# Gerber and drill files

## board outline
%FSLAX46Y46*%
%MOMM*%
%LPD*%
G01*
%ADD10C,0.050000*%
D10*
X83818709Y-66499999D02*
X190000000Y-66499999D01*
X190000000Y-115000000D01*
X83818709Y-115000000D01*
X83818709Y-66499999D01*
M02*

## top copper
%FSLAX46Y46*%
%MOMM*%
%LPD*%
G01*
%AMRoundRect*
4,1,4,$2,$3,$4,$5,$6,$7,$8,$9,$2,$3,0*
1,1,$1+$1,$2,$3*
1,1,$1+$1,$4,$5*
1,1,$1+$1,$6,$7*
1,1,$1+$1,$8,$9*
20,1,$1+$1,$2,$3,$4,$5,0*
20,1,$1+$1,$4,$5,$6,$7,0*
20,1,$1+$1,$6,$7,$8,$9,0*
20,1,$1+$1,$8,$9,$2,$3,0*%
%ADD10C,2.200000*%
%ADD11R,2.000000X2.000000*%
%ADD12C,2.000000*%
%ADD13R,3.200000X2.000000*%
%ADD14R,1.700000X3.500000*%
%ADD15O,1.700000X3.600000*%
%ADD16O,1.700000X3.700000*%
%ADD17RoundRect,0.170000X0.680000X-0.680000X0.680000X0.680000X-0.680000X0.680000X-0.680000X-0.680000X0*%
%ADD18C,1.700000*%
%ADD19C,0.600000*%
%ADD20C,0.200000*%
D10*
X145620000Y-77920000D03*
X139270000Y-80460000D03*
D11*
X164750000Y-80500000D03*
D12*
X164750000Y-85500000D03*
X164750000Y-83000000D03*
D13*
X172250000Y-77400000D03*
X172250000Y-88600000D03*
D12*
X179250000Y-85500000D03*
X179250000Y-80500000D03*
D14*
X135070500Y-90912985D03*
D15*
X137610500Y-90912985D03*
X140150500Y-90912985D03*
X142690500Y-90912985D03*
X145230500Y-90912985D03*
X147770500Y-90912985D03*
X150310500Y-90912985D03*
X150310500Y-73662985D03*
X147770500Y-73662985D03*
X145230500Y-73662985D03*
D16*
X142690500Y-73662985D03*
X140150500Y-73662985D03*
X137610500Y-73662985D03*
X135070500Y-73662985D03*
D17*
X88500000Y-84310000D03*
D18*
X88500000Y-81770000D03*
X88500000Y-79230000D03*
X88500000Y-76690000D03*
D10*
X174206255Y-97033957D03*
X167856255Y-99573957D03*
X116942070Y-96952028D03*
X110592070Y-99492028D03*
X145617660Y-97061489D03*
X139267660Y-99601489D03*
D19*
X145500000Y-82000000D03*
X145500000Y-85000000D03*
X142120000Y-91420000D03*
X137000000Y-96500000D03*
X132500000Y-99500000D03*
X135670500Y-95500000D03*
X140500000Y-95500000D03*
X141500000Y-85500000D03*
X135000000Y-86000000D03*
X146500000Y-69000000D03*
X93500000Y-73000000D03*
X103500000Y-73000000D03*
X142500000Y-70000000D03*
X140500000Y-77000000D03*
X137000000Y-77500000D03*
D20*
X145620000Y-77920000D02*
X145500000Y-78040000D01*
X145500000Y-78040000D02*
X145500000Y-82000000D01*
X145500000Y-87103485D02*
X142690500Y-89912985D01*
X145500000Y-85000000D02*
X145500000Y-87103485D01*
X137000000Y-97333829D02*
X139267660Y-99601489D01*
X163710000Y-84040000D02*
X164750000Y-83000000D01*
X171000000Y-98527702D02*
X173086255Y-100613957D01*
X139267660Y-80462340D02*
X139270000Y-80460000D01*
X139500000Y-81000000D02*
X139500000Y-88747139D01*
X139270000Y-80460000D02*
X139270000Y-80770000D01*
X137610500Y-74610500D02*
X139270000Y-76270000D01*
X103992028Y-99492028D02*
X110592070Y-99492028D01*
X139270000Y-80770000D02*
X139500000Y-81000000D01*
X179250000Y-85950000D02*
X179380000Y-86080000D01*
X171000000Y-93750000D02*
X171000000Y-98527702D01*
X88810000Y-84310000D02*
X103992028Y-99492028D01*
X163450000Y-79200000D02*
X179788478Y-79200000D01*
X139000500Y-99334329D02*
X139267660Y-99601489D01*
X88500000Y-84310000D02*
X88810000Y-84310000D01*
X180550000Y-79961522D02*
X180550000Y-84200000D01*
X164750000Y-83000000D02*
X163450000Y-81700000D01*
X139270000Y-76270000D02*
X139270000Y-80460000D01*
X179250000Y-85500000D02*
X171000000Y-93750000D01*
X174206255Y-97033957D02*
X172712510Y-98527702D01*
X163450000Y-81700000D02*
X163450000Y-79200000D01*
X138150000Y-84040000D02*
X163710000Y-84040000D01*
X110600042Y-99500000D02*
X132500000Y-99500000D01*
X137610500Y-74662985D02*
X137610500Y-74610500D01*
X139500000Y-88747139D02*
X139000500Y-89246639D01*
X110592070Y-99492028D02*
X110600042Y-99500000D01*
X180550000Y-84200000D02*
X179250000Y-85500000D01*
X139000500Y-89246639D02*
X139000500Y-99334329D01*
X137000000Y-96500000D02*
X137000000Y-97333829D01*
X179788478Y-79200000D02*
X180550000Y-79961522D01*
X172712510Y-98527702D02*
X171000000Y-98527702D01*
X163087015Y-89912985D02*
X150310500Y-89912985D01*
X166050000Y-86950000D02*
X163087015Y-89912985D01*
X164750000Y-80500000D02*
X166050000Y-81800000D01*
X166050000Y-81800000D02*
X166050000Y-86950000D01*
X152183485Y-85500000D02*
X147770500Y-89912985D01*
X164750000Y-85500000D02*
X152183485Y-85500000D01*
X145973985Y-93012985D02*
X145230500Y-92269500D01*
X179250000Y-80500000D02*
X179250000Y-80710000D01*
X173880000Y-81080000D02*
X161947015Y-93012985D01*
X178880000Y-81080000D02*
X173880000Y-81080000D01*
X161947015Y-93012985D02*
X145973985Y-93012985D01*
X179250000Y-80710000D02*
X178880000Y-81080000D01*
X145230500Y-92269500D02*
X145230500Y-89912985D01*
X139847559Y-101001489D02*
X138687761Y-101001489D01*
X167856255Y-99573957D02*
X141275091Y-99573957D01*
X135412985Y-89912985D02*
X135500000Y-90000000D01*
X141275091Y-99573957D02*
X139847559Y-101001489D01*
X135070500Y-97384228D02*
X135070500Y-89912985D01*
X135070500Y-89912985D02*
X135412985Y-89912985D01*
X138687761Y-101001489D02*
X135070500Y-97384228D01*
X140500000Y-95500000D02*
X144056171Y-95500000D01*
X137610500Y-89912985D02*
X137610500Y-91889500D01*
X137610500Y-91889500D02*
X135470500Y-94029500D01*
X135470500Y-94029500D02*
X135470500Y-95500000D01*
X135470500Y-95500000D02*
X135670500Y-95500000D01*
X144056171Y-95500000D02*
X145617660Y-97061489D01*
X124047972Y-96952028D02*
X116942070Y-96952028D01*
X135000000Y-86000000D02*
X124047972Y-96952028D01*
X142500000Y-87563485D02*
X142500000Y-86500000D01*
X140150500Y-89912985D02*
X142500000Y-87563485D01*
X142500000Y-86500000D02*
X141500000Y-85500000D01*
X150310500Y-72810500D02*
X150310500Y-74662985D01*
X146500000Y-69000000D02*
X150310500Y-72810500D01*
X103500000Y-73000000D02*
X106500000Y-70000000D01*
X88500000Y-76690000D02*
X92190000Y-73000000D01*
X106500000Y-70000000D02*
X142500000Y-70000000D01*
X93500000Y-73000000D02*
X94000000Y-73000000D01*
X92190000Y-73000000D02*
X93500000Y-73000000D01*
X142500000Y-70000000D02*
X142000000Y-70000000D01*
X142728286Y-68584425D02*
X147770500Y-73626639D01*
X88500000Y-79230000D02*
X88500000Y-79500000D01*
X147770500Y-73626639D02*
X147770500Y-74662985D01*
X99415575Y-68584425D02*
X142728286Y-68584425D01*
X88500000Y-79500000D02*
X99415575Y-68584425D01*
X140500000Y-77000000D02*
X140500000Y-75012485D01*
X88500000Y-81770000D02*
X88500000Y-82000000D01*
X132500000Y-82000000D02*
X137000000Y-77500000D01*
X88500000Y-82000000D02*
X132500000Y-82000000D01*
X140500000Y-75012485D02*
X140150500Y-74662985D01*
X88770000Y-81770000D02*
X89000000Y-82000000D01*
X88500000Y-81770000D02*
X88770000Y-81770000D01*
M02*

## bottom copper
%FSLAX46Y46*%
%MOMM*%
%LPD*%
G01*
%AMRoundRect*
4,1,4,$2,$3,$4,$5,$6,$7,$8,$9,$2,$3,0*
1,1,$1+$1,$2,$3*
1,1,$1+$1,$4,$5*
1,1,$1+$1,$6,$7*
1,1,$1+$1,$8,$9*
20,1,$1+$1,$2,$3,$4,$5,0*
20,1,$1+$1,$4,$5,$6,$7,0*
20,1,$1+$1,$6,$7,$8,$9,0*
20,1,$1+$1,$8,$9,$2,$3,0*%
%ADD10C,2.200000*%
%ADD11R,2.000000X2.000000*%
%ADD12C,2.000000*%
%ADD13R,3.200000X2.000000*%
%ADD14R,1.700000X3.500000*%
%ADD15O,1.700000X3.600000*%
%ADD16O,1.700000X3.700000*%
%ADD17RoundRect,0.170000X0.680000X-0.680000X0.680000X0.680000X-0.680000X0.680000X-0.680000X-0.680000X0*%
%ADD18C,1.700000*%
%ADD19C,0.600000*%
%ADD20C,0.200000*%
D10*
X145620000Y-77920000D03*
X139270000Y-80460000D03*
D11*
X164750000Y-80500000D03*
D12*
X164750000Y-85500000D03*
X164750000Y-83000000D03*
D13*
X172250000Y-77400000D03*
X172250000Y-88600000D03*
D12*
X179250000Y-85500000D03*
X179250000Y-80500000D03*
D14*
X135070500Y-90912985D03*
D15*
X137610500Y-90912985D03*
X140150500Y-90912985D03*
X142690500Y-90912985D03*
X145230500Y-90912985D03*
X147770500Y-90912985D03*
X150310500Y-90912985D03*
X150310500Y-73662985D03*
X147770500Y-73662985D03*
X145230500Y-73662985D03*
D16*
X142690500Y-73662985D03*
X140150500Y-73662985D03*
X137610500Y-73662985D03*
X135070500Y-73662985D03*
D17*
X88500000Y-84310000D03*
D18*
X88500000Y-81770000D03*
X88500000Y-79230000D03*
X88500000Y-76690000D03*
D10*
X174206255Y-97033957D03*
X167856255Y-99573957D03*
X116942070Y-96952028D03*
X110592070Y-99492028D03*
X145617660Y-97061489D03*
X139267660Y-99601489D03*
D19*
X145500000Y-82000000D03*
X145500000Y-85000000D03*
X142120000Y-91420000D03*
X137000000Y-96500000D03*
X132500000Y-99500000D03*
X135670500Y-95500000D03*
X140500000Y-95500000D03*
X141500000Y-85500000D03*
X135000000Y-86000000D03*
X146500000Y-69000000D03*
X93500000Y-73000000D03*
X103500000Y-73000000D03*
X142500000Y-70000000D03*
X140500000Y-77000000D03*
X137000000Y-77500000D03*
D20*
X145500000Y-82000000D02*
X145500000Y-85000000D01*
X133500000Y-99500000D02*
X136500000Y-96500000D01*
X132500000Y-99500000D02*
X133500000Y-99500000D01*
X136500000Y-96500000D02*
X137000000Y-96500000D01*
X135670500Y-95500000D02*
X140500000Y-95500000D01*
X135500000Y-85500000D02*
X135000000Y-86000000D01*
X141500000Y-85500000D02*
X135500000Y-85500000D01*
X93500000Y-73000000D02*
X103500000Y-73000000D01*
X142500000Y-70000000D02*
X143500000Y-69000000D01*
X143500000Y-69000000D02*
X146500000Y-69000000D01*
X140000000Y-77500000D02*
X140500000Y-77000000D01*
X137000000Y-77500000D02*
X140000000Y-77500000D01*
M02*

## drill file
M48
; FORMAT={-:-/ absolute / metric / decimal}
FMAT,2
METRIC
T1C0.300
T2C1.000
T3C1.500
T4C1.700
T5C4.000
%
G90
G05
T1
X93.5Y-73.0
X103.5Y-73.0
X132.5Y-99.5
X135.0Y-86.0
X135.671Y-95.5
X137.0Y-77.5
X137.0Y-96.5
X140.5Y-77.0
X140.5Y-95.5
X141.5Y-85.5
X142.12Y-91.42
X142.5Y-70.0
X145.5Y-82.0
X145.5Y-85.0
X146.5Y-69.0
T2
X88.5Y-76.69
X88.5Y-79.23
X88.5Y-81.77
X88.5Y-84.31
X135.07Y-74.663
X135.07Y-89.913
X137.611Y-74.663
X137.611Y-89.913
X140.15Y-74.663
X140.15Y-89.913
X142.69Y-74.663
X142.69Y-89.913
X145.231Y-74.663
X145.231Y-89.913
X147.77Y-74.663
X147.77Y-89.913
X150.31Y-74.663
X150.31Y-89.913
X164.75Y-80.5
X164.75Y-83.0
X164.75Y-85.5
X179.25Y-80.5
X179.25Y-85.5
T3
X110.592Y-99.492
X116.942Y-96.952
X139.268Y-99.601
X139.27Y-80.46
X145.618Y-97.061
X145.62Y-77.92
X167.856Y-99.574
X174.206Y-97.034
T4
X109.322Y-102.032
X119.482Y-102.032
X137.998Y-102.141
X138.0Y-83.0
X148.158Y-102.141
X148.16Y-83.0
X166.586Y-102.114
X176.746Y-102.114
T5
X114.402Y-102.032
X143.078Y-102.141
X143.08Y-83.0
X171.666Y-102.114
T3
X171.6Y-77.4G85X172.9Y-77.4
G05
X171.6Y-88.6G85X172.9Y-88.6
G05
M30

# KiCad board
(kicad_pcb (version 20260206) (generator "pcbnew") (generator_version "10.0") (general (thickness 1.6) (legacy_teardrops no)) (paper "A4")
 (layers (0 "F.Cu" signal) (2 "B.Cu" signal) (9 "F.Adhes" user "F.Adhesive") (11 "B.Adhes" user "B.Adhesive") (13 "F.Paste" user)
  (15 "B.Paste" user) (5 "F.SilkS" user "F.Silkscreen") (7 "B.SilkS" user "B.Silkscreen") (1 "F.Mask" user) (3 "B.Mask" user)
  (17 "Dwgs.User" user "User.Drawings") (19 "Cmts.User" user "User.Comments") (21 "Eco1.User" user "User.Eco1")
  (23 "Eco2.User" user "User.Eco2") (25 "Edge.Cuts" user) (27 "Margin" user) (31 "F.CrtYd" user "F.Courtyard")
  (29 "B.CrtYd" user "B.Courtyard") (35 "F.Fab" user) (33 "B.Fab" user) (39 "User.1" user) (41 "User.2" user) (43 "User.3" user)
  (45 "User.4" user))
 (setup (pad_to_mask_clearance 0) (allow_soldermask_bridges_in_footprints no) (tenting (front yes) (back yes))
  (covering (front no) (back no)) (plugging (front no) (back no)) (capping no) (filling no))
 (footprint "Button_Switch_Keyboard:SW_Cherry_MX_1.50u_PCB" (layer "F.Cu") (at 145.62 77.92)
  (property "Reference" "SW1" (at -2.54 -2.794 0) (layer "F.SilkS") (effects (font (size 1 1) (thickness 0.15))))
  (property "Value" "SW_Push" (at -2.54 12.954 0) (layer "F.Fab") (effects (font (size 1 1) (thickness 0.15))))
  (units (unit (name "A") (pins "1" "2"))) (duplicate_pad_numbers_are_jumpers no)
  (pad "" np_thru_hole circle (at -7.62 5.08) (size 1.7 1.7) (drill 1.7) (layers "*.Cu" "*.Mask"))
  (pad "" np_thru_hole circle (at -2.54 5.08) (size 4 4) (drill 4) (layers "*.Cu" "*.Mask"))
  (pad "" np_thru_hole circle (at 2.54 5.08) (size 1.7 1.7) (drill 1.7) (layers "*.Cu" "*.Mask"))
  (pad "1" thru_hole circle (at 0 0) (size 2.2 2.2) (drill 1.5) (layers "*.Cu" "*.Mask") (remove_unused_layers no)
   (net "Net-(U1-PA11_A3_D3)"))
  (pad "2" thru_hole circle (at -6.35 2.54) (size 2.2 2.2) (drill 1.5) (layers "*.Cu" "*.Mask") (remove_unused_layers no) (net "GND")))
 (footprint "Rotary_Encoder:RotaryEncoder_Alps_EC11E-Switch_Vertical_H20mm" (layer "F.Cu") (at 164.75 80.5)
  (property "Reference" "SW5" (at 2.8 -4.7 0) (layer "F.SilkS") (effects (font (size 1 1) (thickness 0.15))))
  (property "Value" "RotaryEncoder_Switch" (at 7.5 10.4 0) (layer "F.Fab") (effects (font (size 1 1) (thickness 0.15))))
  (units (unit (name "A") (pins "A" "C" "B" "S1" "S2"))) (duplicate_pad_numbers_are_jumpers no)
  (pad "A" thru_hole rect (at 0 0) (size 2 2) (drill 1) (layers "*.Cu" "*.Mask") (remove_unused_layers no) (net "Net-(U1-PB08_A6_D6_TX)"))
  (pad "B" thru_hole circle (at 0 5) (size 2 2) (drill 1) (layers "*.Cu" "*.Mask") (remove_unused_layers no) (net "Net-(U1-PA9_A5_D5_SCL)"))
  (pad "C" thru_hole circle (at 0 2.5) (size 2 2) (drill 1) (layers "*.Cu" "*.Mask") (remove_unused_layers no) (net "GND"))
  (pad "MP" thru_hole rect (at 7.5 -3.1) (size 3.2 2) (drill oval 2.8 1.5) (layers "*.Cu" "*.Mask") (remove_unused_layers no))
  (pad "MP" thru_hole rect (at 7.5 8.1) (size 3.2 2) (drill oval 2.8 1.5) (layers "*.Cu" "*.Mask") (remove_unused_layers no))
  (pad "S1" thru_hole circle (at 14.5 5) (size 2 2) (drill 1) (layers "*.Cu" "*.Mask") (remove_unused_layers no) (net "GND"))
  (pad "S2" thru_hole circle (at 14.5 0) (size 2 2) (drill 1) (layers "*.Cu" "*.Mask") (remove_unused_layers no)
   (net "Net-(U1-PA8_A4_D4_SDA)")))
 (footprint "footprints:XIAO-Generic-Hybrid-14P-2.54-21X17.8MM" (layer "F.Cu") (at 142.6905 82.287985 90)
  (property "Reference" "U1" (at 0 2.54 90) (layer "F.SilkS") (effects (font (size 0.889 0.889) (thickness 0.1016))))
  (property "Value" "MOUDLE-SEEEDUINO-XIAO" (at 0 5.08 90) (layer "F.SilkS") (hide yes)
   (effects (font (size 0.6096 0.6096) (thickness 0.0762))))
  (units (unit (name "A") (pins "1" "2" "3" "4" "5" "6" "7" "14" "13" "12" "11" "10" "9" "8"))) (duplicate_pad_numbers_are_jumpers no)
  (pad "1" thru_hole rect (at -7.625 -7.62 90) (size 3.5 1.7) (drill 1 (offset -1 0)) (layers "*.Cu" "*.Mask") (remove_unused_layers no)
   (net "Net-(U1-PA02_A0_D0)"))
  (pad "2" thru_hole oval (at -7.625 -5.08 90) (size 3.6 1.7) (drill 1 (offset -1 0)) (layers "*.Cu" "*.Mask") (remove_unused_layers no)
   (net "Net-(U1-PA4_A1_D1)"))
  (pad "3" thru_hole oval (at -7.625 -2.54 90) (size 3.6 1.7) (drill 1 (offset -1 0)) (layers "*.Cu" "*.Mask") (remove_unused_layers no)
   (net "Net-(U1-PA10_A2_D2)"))
  (pad "4" thru_hole oval (at -7.625 0 90) (size 3.6 1.7) (drill 1 (offset -1 0)) (layers "*.Cu" "*.Mask") (remove_unused_layers no)
   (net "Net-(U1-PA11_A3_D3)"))
  (pad "5" thru_hole oval (at -7.625 2.54 90) (size 3.6 1.7) (drill 1 (offset -1 0)) (layers "*.Cu" "*.Mask") (remove_unused_layers no)
   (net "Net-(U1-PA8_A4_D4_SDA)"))
  (pad "6" thru_hole oval (at -7.625 5.08 270) (size 3.6 1.7) (drill 1 (offset 1 0)) (layers "*.Cu" "*.Mask") (remove_unused_layers no)
   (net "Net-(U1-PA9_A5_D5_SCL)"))
  (pad "7" thru_hole oval (at -7.625 7.62 90) (size 3.6 1.7) (drill 1 (offset -1 0)) (layers "*.Cu" "*.Mask") (remove_unused_layers no)
   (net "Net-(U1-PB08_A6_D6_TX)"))
  (pad "8" thru_hole oval (at 7.625 7.62 90) (size 3.6 1.7) (drill 1 (offset 1 0)) (layers "*.Cu" "*.Mask") (remove_unused_layers no)
   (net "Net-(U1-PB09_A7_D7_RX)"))
  (pad "9" thru_hole oval (at 7.625 5.08 90) (size 3.6 1.7) (drill 1 (offset 1 0)) (layers "*.Cu" "*.Mask") (remove_unused_layers no)
   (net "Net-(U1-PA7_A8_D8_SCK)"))
  (pad "10" thru_hole oval (at 7.625 2.54 90) (size 3.6 1.7) (drill 1 (offset 1 0)) (layers "*.Cu" "*.Mask") (remove_unused_layers no)
   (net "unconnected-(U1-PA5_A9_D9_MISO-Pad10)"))
  (pad "11" thru_hole oval (at 7.625 0 90) (size 3.7 1.7) (drill 1 (offset 1 0)) (layers "*.Cu" "*.Mask") (remove_unused_layers no)
   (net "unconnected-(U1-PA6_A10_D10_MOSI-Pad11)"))
  (pad "12" thru_hole oval (at 7.625 -2.54 90) (size 3.7 1.7) (drill 1 (offset 1 0)) (layers "*.Cu" "*.Mask") (remove_unused_layers no)
   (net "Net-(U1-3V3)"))
  (pad "13" thru_hole oval (at 7.625 -5.08 90) (size 3.7 1.7) (drill 1 (offset 1 0)) (layers "*.Cu" "*.Mask") (remove_unused_layers no)
   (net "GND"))
  (pad "14" thru_hole oval (at 7.625 -7.62 90) (size 3.7 1.7) (drill 1 (offset 1 0)) (layers "*.Cu" "*.Mask") (remove_unused_layers no)
   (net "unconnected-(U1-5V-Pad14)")))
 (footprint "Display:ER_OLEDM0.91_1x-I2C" (layer "F.Cu") (at 88.5 84.31 90)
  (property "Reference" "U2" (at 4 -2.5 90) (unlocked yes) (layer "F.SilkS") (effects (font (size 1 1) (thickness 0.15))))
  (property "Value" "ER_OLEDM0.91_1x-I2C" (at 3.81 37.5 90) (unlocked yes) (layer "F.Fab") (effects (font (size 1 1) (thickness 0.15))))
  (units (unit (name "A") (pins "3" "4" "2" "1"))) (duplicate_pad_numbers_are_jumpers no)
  (pad "1" thru_hole roundrect (at 0 0 90) (size 1.7 1.7) (drill 1) (layers "*.Cu" "*.Mask") (remove_unused_layers no)
   (roundrect_rratio 0.1) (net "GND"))
  (pad "2" thru_hole circle (at 2.54 0 90) (size 1.7 1.7) (drill 1) (layers "*.Cu" "*.Mask") (remove_unused_layers no) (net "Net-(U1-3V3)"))
  (pad "3" thru_hole circle (at 5.08 0 90) (size 1.7 1.7) (drill 1) (layers "*.Cu" "*.Mask") (remove_unused_layers no)
   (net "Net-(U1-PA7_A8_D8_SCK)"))
  (pad "4" thru_hole circle (at 7.62 0 90) (size 1.7 1.7) (drill 1) (layers "*.Cu" "*.Mask") (remove_unused_layers no)
   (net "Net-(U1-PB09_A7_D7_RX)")))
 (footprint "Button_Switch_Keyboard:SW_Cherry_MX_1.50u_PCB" (layer "F.Cu") (at 174.206255 97.033957)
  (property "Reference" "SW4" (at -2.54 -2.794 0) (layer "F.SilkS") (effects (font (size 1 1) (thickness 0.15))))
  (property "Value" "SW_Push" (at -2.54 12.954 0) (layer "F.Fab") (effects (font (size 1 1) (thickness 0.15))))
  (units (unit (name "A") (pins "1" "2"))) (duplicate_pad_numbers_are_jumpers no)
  (pad "" np_thru_hole circle (at -7.62 5.08) (size 1.7 1.7) (drill 1.7) (layers "*.Cu" "*.Mask"))
  (pad "" np_thru_hole circle (at -2.54 5.08) (size 4 4) (drill 4) (layers "*.Cu" "*.Mask"))
  (pad "" np_thru_hole circle (at 2.54 5.08) (size 1.7 1.7) (drill 1.7) (layers "*.Cu" "*.Mask"))
  (pad "1" thru_hole circle (at 0 0) (size 2.2 2.2) (drill 1.5) (layers "*.Cu" "*.Mask") (remove_unused_layers no) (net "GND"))
  (pad "2" thru_hole circle (at -6.35 2.54) (size 2.2 2.2) (drill 1.5) (layers "*.Cu" "*.Mask") (remove_unused_layers no)
   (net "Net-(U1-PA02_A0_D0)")))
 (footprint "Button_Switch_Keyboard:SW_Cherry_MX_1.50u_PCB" (layer "F.Cu") (at 116.94207 96.952028)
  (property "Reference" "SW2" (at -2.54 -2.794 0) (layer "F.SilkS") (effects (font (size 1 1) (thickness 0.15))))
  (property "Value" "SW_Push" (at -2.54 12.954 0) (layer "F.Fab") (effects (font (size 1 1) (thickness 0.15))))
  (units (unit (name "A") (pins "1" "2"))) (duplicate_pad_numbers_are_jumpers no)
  (pad "" np_thru_hole circle (at -7.62 5.08) (size 1.7 1.7) (drill 1.7) (layers "*.Cu" "*.Mask"))
  (pad "" np_thru_hole circle (at -2.54 5.08) (size 4 4) (drill 4) (layers "*.Cu" "*.Mask"))
  (pad "" np_thru_hole circle (at 2.54 5.08) (size 1.7 1.7) (drill 1.7) (layers "*.Cu" "*.Mask"))
  (pad "1" thru_hole circle (at 0 0) (size 2.2 2.2) (drill 1.5) (layers "*.Cu" "*.Mask") (remove_unused_layers no)
   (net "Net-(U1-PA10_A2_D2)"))
  (pad "2" thru_hole circle (at -6.35 2.54) (size 2.2 2.2) (drill 1.5) (layers "*.Cu" "*.Mask") (remove_unused_layers no) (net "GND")))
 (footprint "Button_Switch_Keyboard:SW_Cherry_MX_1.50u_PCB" (layer "F.Cu") (at 145.61766 97.061489)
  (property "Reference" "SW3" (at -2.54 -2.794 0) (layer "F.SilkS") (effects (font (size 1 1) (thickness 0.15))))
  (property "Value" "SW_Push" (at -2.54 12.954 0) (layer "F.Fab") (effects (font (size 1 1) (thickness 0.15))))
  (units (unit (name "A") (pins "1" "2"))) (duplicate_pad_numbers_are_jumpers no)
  (pad "" np_thru_hole circle (at -7.62 5.08) (size 1.7 1.7) (drill 1.7) (layers "*.Cu" "*.Mask"))
  (pad "" np_thru_hole circle (at -2.54 5.08) (size 4 4) (drill 4) (layers "*.Cu" "*.Mask"))
  (pad "" np_thru_hole circle (at 2.54 5.08) (size 1.7 1.7) (drill 1.7) (layers "*.Cu" "*.Mask"))
  (pad "1" thru_hole circle (at 0 0) (size 2.2 2.2) (drill 1.5) (layers "*.Cu" "*.Mask") (remove_unused_layers no)
   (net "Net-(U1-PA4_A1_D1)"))
  (pad "2" thru_hole circle (at -6.35 2.54) (size 2.2 2.2) (drill 1.5) (layers "*.Cu" "*.Mask") (remove_unused_layers no) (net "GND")))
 (gr_rect (start 83.818709 66.499999) (end 190 115) (stroke (width 0.05) (type default)) (fill no) (layer "Edge.Cuts"))
 (segment (start 145.62 77.92) (end 145.5 78.04) (width 0.2) (layer "F.Cu") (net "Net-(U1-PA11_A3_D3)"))
 (segment (start 145.5 78.04) (end 145.5 82) (width 0.2) (layer "F.Cu") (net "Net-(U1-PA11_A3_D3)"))
 (segment (start 145.5 87.103485) (end 142.6905 89.912985) (width 0.2) (layer "F.Cu") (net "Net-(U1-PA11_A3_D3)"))
 (segment (start 145.5 85) (end 145.5 87.103485) (width 0.2) (layer "F.Cu") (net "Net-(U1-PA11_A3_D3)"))
 (via (at 145.5 82) (size 0.6) (drill 0.3) (layers "F.Cu" "B.Cu") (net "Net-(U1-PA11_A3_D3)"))
 (via (at 145.5 85) (size 0.6) (drill 0.3) (layers "F.Cu" "B.Cu") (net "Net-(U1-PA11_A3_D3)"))
 (via (at 142.12 91.42) (size 0.6) (drill 0.3) (layers "F.Cu" "B.Cu") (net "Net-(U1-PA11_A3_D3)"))
 (segment (start 145.5 82) (end 145.5 85) (width 0.2) (layer "B.Cu") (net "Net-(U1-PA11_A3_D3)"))
 (segment (start 137 97.333829) (end 139.26766 99.601489) (width 0.2) (layer "F.Cu") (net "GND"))
 (segment (start 163.71 84.04) (end 164.75 83) (width 0.2) (layer "F.Cu") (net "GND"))
 (segment (start 171 98.527702) (end 173.086255 100.613957) (width 0.2) (layer "F.Cu") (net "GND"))
 (segment (start 139.26766 80.46234) (end 139.27 80.46) (width 0.2) (layer "F.Cu") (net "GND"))
 (segment (start 139.5 81) (end 139.5 88.747139) (width 0.2) (layer "F.Cu") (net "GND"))
 (segment (start 139.27 80.46) (end 139.27 80.77) (width 0.2) (layer "F.Cu") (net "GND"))
 (segment (start 137.6105 74.6105) (end 139.27 76.27) (width 0.2) (layer "F.Cu") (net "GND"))
 (segment (start 103.992028 99.492028) (end 110.59207 99.492028) (width 0.2) (layer "F.Cu") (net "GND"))
 (segment (start 139.27 80.77) (end 139.5 81) (width 0.2) (layer "F.Cu") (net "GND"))
 (segment (start 179.25 85.95) (end 179.38 86.08) (width 0.2) (layer "F.Cu") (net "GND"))
 (segment (start 171 93.75) (end 171 98.527702) (width 0.2) (layer "F.Cu") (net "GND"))
 (segment (start 88.81 84.31) (end 103.992028 99.492028) (width 0.2) (layer "F.Cu") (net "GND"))
 (segment (start 163.45 79.2) (end 179.788478 79.2) (width 0.2) (layer "F.Cu") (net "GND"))
 (segment (start 139.0005 99.334329) (end 139.26766 99.601489) (width 0.2) (layer "F.Cu") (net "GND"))
 (segment (start 88.5 84.31) (end 88.81 84.31) (width 0.2) (layer "F.Cu") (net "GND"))
 (segment (start 180.55 79.961522) (end 180.55 84.2) (width 0.2) (layer "F.Cu") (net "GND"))
 (segment (start 164.75 83) (end 163.45 81.7) (width 0.2) (layer "F.Cu") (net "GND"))
 (segment (start 139.27 76.27) (end 139.27 80.46) (width 0.2) (layer "F.Cu") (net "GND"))
 (segment (start 179.25 85.5) (end 171 93.75) (width 0.2) (layer "F.Cu") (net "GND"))
 (segment (start 174.206255 97.033957) (end 172.71251 98.527702) (width 0.2) (layer "F.Cu") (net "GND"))
 (segment (start 163.45 81.7) (end 163.45 79.2) (width 0.2) (layer "F.Cu") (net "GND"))
 (segment (start 138.15 84.04) (end 163.71 84.04) (width 0.2) (layer "F.Cu") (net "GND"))
 (segment (start 110.600042 99.5) (end 132.5 99.5) (width 0.2) (layer "F.Cu") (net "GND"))
 (segment (start 137.6105 74.662985) (end 137.6105 74.6105) (width 0.2) (layer "F.Cu") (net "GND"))
 (segment (start 139.5 88.747139) (end 139.0005 89.246639) (width 0.2) (layer "F.Cu") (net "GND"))
 (segment (start 110.59207 99.492028) (end 110.600042 99.5) (width 0.2) (layer "F.Cu") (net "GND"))
 (segment (start 180.55 84.2) (end 179.25 85.5) (width 0.2) (layer "F.Cu") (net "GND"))
 (segment (start 139.0005 89.246639) (end 139.0005 99.334329) (width 0.2) (layer "F.Cu") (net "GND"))
 (segment (start 137 96.5) (end 137 97.333829) (width 0.2) (layer "F.Cu") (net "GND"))
 (segment (start 179.788478 79.2) (end 180.55 79.961522) (width 0.2) (layer "F.Cu") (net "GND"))
 (segment (start 172.71251 98.527702) (end 171 98.527702) (width 0.2) (layer "F.Cu") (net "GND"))
 (via (at 137 96.5) (size 0.6) (drill 0.3) (layers "F.Cu" "B.Cu") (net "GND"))
 (via (at 132.5 99.5) (size 0.6) (drill 0.3) (layers "F.Cu" "B.Cu") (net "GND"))
 (segment (start 133.5 99.5) (end 136.5 96.5) (width 0.2) (layer "B.Cu") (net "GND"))
 (segment (start 132.5 99.5) (end 133.5 99.5) (width 0.2) (layer "B.Cu") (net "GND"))
 (segment (start 136.5 96.5) (end 137 96.5) (width 0.2) (layer "B.Cu") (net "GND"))
 (segment (start 163.087015 89.912985) (end 150.3105 89.912985) (width 0.2) (layer "F.Cu") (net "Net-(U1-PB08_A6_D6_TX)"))
 (segment (start 166.05 86.95) (end 163.087015 89.912985) (width 0.2) (layer "F.Cu") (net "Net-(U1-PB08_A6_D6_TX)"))
 (segment (start 164.75 80.5) (end 166.05 81.8) (width 0.2) (layer "F.Cu") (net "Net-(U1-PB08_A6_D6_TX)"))
 (segment (start 166.05 81.8) (end 166.05 86.95) (width 0.2) (layer "F.Cu") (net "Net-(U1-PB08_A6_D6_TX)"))
 (segment (start 152.183485 85.5) (end 147.7705 89.912985) (width 0.2) (layer "F.Cu") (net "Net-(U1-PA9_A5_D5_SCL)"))
 (segment (start 164.75 85.5) (end 152.183485 85.5) (width 0.2) (layer "F.Cu") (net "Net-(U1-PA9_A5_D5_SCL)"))
 (segment (start 145.973985 93.012985) (end 145.2305 92.2695) (width 0.2) (layer "F.Cu") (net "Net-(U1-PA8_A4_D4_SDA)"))
 (segment (start 179.25 80.5) (end 179.25 80.71) (width 0.2) (layer "F.Cu") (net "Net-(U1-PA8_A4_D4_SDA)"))
 (segment (start 173.88 81.08) (end 161.947015 93.012985) (width 0.2) (layer "F.Cu") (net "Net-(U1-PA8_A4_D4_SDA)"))
 (segment (start 178.88 81.08) (end 173.88 81.08) (width 0.2) (layer "F.Cu") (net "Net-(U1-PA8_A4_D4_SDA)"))
 (segment (start 161.947015 93.012985) (end 145.973985 93.012985) (width 0.2) (layer "F.Cu") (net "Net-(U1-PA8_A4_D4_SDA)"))
 (segment (start 179.25 80.71) (end 178.88 81.08) (width 0.2) (layer "F.Cu") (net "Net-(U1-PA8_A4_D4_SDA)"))
 (segment (start 145.2305 92.2695) (end 145.2305 89.912985) (width 0.2) (layer "F.Cu") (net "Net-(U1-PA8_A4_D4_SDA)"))
 (segment (start 139.847559 101.001489) (end 138.687761 101.001489) (width 0.2) (layer "F.Cu") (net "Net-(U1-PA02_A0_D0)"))
 (segment (start 167.856255 99.573957) (end 141.275091 99.573957) (width 0.2) (layer "F.Cu") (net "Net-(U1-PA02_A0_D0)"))
 (segment (start 135.412985 89.912985) (end 135.5 90) (width 0.2) (layer "F.Cu") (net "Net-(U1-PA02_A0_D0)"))
 (segment (start 141.275091 99.573957) (end 139.847559 101.001489) (width 0.2) (layer "F.Cu") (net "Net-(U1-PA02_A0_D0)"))
 (segment (start 135.0705 97.384228) (end 135.0705 89.912985) (width 0.2) (layer "F.Cu") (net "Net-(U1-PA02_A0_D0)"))
 (segment (start 135.0705 89.912985) (end 135.412985 89.912985) (width 0.2) (layer "F.Cu") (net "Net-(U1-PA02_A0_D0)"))
 (segment (start 138.687761 101.001489) (end 135.0705 97.384228) (width 0.2) (layer "F.Cu") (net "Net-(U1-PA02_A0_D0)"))
 (segment (start 140.5 95.5) (end 144.056171 95.5) (width 0.2) (layer "F.Cu") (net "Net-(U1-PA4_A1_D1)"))
 (segment (start 137.6105 89.912985) (end 137.6105 91.8895) (width 0.2) (layer "F.Cu") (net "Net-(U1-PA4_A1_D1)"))
 (segment (start 137.6105 91.8895) (end 135.4705 94.0295) (width 0.2) (layer "F.Cu") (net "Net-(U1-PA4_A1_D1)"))
 (segment (start 135.4705 94.0295) (end 135.4705 95.5) (width 0.2) (layer "F.Cu") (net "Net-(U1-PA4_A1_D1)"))
 (segment (start 135.4705 95.5) (end 135.6705 95.5) (width 0.2) (layer "F.Cu") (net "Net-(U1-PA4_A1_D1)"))
 (segment (start 144.056171 95.5) (end 145.61766 97.061489) (width 0.2) (layer "F.Cu") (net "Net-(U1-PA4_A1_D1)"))
 (via (at 135.6705 95.5) (size 0.6) (drill 0.3) (layers "F.Cu" "B.Cu") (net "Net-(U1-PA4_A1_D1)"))
 (via (at 140.5 95.5) (size 0.6) (drill 0.3) (layers "F.Cu" "B.Cu") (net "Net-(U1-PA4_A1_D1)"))
 (segment (start 135.6705 95.5) (end 140.5 95.5) (width 0.2) (layer "B.Cu") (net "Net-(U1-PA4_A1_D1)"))
 (segment (start 124.047972 96.952028) (end 116.94207 96.952028) (width 0.2) (layer "F.Cu") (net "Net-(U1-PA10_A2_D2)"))
 (segment (start 135 86) (end 124.047972 96.952028) (width 0.2) (layer "F.Cu") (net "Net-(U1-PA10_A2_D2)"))
 (segment (start 142.5 87.563485) (end 142.5 86.5) (width 0.2) (layer "F.Cu") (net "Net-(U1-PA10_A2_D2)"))
 (segment (start 140.1505 89.912985) (end 142.5 87.563485) (width 0.2) (layer "F.Cu") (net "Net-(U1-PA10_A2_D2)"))
 (segment (start 142.5 86.5) (end 141.5 85.5) (width 0.2) (layer "F.Cu") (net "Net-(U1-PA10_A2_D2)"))
 (via (at 141.5 85.5) (size 0.6) (drill 0.3) (layers "F.Cu" "B.Cu") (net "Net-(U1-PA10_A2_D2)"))
 (via (at 135 86) (size 0.6) (drill 0.3) (layers "F.Cu" "B.Cu") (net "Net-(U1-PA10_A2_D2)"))
 (segment (start 135.5 85.5) (end 135 86) (width 0.2) (layer "B.Cu") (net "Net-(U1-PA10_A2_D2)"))
 (segment (start 141.5 85.5) (end 135.5 85.5) (width 0.2) (layer "B.Cu") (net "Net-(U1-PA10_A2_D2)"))
 (segment (start 150.3105 72.8105) (end 150.3105 74.662985) (width 0.2) (layer "F.Cu") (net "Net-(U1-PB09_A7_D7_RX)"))
 (segment (start 146.5 69) (end 150.3105 72.8105) (width 0.2) (layer "F.Cu") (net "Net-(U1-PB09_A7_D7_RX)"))
 (segment (start 103.5 73) (end 106.5 70) (width 0.2) (layer "F.Cu") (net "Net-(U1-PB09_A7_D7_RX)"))
 (segment (start 88.5 76.69) (end 92.19 73) (width 0.2) (layer "F.Cu") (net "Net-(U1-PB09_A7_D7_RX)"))
 (segment (start 106.5 70) (end 142.5 70) (width 0.2) (layer "F.Cu") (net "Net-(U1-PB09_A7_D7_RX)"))
 (segment (start 93.5 73) (end 94 73) (width 0.2) (layer "F.Cu") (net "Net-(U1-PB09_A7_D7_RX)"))
 (segment (start 92.19 73) (end 93.5 73) (width 0.2) (layer "F.Cu") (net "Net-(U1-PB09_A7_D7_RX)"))
 (segment (start 142.5 70) (end 142 70) (width 0.2) (layer "F.Cu") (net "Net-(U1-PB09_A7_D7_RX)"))
 (via (at 146.5 69) (size 0.6) (drill 0.3) (layers "F.Cu" "B.Cu") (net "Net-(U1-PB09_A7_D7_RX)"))
 (via (at 93.5 73) (size 0.6) (drill 0.3) (layers "F.Cu" "B.Cu") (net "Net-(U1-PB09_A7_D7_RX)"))
 (via (at 103.5 73) (size 0.6) (drill 0.3) (layers "F.Cu" "B.Cu") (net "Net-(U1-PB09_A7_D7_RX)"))
 (via (at 142.5 70) (size 0.6) (drill 0.3) (layers "F.Cu" "B.Cu") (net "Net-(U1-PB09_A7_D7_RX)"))
 (segment (start 93.5 73) (end 103.5 73) (width 0.2) (layer "B.Cu") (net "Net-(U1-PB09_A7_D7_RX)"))
 (segment (start 142.5 70) (end 143.5 69) (width 0.2) (layer "B.Cu") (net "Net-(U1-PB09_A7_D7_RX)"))
 (segment (start 143.5 69) (end 146.5 69) (width 0.2) (layer "B.Cu") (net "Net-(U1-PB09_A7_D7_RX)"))
 (segment (start 142.728286 68.584425) (end 147.7705 73.626639) (width 0.2) (layer "F.Cu") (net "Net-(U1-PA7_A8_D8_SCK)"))
 (segment (start 88.5 79.23) (end 88.5 79.5) (width 0.2) (layer "F.Cu") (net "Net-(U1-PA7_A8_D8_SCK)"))
 (segment (start 147.7705 73.626639) (end 147.7705 74.662985) (width 0.2) (layer "F.Cu") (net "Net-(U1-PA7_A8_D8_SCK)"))
 (segment (start 99.415575 68.584425) (end 142.728286 68.584425) (width 0.2) (layer "F.Cu") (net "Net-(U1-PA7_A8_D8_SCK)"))
 (segment (start 88.5 79.5) (end 99.415575 68.584425) (width 0.2) (layer "F.Cu") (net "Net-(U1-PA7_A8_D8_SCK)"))
 (segment (start 140.5 77) (end 140.5 75.012485) (width 0.2) (layer "F.Cu") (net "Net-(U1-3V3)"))
 (segment (start 88.5 81.77) (end 88.5 82) (width 0.2) (layer "F.Cu") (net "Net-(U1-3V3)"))
 (segment (start 132.5 82) (end 137 77.5) (width 0.2) (layer "F.Cu") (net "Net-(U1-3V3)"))
 (segment (start 88.5 82) (end 132.5 82) (width 0.2) (layer "F.Cu") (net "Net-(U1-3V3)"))
 (segment (start 140.5 75.012485) (end 140.1505 74.662985) (width 0.2) (layer "F.Cu") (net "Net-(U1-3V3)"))
 (segment (start 88.77 81.77) (end 89 82) (width 0.2) (layer "F.Cu") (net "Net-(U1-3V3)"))
 (segment (start 88.5 81.77) (end 88.77 81.77) (width 0.2) (layer "F.Cu") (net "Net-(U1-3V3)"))
 (via (at 140.5 77) (size 0.6) (drill 0.3) (layers "F.Cu" "B.Cu") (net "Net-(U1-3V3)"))
 (via (at 137 77.5) (size 0.6) (drill 0.3) (layers "F.Cu" "B.Cu") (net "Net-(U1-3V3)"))
 (segment (start 140 77.5) (end 140.5 77) (width 0.2) (layer "B.Cu") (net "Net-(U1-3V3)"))
 (segment (start 137 77.5) (end 140 77.5) (width 0.2) (layer "B.Cu") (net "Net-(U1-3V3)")))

